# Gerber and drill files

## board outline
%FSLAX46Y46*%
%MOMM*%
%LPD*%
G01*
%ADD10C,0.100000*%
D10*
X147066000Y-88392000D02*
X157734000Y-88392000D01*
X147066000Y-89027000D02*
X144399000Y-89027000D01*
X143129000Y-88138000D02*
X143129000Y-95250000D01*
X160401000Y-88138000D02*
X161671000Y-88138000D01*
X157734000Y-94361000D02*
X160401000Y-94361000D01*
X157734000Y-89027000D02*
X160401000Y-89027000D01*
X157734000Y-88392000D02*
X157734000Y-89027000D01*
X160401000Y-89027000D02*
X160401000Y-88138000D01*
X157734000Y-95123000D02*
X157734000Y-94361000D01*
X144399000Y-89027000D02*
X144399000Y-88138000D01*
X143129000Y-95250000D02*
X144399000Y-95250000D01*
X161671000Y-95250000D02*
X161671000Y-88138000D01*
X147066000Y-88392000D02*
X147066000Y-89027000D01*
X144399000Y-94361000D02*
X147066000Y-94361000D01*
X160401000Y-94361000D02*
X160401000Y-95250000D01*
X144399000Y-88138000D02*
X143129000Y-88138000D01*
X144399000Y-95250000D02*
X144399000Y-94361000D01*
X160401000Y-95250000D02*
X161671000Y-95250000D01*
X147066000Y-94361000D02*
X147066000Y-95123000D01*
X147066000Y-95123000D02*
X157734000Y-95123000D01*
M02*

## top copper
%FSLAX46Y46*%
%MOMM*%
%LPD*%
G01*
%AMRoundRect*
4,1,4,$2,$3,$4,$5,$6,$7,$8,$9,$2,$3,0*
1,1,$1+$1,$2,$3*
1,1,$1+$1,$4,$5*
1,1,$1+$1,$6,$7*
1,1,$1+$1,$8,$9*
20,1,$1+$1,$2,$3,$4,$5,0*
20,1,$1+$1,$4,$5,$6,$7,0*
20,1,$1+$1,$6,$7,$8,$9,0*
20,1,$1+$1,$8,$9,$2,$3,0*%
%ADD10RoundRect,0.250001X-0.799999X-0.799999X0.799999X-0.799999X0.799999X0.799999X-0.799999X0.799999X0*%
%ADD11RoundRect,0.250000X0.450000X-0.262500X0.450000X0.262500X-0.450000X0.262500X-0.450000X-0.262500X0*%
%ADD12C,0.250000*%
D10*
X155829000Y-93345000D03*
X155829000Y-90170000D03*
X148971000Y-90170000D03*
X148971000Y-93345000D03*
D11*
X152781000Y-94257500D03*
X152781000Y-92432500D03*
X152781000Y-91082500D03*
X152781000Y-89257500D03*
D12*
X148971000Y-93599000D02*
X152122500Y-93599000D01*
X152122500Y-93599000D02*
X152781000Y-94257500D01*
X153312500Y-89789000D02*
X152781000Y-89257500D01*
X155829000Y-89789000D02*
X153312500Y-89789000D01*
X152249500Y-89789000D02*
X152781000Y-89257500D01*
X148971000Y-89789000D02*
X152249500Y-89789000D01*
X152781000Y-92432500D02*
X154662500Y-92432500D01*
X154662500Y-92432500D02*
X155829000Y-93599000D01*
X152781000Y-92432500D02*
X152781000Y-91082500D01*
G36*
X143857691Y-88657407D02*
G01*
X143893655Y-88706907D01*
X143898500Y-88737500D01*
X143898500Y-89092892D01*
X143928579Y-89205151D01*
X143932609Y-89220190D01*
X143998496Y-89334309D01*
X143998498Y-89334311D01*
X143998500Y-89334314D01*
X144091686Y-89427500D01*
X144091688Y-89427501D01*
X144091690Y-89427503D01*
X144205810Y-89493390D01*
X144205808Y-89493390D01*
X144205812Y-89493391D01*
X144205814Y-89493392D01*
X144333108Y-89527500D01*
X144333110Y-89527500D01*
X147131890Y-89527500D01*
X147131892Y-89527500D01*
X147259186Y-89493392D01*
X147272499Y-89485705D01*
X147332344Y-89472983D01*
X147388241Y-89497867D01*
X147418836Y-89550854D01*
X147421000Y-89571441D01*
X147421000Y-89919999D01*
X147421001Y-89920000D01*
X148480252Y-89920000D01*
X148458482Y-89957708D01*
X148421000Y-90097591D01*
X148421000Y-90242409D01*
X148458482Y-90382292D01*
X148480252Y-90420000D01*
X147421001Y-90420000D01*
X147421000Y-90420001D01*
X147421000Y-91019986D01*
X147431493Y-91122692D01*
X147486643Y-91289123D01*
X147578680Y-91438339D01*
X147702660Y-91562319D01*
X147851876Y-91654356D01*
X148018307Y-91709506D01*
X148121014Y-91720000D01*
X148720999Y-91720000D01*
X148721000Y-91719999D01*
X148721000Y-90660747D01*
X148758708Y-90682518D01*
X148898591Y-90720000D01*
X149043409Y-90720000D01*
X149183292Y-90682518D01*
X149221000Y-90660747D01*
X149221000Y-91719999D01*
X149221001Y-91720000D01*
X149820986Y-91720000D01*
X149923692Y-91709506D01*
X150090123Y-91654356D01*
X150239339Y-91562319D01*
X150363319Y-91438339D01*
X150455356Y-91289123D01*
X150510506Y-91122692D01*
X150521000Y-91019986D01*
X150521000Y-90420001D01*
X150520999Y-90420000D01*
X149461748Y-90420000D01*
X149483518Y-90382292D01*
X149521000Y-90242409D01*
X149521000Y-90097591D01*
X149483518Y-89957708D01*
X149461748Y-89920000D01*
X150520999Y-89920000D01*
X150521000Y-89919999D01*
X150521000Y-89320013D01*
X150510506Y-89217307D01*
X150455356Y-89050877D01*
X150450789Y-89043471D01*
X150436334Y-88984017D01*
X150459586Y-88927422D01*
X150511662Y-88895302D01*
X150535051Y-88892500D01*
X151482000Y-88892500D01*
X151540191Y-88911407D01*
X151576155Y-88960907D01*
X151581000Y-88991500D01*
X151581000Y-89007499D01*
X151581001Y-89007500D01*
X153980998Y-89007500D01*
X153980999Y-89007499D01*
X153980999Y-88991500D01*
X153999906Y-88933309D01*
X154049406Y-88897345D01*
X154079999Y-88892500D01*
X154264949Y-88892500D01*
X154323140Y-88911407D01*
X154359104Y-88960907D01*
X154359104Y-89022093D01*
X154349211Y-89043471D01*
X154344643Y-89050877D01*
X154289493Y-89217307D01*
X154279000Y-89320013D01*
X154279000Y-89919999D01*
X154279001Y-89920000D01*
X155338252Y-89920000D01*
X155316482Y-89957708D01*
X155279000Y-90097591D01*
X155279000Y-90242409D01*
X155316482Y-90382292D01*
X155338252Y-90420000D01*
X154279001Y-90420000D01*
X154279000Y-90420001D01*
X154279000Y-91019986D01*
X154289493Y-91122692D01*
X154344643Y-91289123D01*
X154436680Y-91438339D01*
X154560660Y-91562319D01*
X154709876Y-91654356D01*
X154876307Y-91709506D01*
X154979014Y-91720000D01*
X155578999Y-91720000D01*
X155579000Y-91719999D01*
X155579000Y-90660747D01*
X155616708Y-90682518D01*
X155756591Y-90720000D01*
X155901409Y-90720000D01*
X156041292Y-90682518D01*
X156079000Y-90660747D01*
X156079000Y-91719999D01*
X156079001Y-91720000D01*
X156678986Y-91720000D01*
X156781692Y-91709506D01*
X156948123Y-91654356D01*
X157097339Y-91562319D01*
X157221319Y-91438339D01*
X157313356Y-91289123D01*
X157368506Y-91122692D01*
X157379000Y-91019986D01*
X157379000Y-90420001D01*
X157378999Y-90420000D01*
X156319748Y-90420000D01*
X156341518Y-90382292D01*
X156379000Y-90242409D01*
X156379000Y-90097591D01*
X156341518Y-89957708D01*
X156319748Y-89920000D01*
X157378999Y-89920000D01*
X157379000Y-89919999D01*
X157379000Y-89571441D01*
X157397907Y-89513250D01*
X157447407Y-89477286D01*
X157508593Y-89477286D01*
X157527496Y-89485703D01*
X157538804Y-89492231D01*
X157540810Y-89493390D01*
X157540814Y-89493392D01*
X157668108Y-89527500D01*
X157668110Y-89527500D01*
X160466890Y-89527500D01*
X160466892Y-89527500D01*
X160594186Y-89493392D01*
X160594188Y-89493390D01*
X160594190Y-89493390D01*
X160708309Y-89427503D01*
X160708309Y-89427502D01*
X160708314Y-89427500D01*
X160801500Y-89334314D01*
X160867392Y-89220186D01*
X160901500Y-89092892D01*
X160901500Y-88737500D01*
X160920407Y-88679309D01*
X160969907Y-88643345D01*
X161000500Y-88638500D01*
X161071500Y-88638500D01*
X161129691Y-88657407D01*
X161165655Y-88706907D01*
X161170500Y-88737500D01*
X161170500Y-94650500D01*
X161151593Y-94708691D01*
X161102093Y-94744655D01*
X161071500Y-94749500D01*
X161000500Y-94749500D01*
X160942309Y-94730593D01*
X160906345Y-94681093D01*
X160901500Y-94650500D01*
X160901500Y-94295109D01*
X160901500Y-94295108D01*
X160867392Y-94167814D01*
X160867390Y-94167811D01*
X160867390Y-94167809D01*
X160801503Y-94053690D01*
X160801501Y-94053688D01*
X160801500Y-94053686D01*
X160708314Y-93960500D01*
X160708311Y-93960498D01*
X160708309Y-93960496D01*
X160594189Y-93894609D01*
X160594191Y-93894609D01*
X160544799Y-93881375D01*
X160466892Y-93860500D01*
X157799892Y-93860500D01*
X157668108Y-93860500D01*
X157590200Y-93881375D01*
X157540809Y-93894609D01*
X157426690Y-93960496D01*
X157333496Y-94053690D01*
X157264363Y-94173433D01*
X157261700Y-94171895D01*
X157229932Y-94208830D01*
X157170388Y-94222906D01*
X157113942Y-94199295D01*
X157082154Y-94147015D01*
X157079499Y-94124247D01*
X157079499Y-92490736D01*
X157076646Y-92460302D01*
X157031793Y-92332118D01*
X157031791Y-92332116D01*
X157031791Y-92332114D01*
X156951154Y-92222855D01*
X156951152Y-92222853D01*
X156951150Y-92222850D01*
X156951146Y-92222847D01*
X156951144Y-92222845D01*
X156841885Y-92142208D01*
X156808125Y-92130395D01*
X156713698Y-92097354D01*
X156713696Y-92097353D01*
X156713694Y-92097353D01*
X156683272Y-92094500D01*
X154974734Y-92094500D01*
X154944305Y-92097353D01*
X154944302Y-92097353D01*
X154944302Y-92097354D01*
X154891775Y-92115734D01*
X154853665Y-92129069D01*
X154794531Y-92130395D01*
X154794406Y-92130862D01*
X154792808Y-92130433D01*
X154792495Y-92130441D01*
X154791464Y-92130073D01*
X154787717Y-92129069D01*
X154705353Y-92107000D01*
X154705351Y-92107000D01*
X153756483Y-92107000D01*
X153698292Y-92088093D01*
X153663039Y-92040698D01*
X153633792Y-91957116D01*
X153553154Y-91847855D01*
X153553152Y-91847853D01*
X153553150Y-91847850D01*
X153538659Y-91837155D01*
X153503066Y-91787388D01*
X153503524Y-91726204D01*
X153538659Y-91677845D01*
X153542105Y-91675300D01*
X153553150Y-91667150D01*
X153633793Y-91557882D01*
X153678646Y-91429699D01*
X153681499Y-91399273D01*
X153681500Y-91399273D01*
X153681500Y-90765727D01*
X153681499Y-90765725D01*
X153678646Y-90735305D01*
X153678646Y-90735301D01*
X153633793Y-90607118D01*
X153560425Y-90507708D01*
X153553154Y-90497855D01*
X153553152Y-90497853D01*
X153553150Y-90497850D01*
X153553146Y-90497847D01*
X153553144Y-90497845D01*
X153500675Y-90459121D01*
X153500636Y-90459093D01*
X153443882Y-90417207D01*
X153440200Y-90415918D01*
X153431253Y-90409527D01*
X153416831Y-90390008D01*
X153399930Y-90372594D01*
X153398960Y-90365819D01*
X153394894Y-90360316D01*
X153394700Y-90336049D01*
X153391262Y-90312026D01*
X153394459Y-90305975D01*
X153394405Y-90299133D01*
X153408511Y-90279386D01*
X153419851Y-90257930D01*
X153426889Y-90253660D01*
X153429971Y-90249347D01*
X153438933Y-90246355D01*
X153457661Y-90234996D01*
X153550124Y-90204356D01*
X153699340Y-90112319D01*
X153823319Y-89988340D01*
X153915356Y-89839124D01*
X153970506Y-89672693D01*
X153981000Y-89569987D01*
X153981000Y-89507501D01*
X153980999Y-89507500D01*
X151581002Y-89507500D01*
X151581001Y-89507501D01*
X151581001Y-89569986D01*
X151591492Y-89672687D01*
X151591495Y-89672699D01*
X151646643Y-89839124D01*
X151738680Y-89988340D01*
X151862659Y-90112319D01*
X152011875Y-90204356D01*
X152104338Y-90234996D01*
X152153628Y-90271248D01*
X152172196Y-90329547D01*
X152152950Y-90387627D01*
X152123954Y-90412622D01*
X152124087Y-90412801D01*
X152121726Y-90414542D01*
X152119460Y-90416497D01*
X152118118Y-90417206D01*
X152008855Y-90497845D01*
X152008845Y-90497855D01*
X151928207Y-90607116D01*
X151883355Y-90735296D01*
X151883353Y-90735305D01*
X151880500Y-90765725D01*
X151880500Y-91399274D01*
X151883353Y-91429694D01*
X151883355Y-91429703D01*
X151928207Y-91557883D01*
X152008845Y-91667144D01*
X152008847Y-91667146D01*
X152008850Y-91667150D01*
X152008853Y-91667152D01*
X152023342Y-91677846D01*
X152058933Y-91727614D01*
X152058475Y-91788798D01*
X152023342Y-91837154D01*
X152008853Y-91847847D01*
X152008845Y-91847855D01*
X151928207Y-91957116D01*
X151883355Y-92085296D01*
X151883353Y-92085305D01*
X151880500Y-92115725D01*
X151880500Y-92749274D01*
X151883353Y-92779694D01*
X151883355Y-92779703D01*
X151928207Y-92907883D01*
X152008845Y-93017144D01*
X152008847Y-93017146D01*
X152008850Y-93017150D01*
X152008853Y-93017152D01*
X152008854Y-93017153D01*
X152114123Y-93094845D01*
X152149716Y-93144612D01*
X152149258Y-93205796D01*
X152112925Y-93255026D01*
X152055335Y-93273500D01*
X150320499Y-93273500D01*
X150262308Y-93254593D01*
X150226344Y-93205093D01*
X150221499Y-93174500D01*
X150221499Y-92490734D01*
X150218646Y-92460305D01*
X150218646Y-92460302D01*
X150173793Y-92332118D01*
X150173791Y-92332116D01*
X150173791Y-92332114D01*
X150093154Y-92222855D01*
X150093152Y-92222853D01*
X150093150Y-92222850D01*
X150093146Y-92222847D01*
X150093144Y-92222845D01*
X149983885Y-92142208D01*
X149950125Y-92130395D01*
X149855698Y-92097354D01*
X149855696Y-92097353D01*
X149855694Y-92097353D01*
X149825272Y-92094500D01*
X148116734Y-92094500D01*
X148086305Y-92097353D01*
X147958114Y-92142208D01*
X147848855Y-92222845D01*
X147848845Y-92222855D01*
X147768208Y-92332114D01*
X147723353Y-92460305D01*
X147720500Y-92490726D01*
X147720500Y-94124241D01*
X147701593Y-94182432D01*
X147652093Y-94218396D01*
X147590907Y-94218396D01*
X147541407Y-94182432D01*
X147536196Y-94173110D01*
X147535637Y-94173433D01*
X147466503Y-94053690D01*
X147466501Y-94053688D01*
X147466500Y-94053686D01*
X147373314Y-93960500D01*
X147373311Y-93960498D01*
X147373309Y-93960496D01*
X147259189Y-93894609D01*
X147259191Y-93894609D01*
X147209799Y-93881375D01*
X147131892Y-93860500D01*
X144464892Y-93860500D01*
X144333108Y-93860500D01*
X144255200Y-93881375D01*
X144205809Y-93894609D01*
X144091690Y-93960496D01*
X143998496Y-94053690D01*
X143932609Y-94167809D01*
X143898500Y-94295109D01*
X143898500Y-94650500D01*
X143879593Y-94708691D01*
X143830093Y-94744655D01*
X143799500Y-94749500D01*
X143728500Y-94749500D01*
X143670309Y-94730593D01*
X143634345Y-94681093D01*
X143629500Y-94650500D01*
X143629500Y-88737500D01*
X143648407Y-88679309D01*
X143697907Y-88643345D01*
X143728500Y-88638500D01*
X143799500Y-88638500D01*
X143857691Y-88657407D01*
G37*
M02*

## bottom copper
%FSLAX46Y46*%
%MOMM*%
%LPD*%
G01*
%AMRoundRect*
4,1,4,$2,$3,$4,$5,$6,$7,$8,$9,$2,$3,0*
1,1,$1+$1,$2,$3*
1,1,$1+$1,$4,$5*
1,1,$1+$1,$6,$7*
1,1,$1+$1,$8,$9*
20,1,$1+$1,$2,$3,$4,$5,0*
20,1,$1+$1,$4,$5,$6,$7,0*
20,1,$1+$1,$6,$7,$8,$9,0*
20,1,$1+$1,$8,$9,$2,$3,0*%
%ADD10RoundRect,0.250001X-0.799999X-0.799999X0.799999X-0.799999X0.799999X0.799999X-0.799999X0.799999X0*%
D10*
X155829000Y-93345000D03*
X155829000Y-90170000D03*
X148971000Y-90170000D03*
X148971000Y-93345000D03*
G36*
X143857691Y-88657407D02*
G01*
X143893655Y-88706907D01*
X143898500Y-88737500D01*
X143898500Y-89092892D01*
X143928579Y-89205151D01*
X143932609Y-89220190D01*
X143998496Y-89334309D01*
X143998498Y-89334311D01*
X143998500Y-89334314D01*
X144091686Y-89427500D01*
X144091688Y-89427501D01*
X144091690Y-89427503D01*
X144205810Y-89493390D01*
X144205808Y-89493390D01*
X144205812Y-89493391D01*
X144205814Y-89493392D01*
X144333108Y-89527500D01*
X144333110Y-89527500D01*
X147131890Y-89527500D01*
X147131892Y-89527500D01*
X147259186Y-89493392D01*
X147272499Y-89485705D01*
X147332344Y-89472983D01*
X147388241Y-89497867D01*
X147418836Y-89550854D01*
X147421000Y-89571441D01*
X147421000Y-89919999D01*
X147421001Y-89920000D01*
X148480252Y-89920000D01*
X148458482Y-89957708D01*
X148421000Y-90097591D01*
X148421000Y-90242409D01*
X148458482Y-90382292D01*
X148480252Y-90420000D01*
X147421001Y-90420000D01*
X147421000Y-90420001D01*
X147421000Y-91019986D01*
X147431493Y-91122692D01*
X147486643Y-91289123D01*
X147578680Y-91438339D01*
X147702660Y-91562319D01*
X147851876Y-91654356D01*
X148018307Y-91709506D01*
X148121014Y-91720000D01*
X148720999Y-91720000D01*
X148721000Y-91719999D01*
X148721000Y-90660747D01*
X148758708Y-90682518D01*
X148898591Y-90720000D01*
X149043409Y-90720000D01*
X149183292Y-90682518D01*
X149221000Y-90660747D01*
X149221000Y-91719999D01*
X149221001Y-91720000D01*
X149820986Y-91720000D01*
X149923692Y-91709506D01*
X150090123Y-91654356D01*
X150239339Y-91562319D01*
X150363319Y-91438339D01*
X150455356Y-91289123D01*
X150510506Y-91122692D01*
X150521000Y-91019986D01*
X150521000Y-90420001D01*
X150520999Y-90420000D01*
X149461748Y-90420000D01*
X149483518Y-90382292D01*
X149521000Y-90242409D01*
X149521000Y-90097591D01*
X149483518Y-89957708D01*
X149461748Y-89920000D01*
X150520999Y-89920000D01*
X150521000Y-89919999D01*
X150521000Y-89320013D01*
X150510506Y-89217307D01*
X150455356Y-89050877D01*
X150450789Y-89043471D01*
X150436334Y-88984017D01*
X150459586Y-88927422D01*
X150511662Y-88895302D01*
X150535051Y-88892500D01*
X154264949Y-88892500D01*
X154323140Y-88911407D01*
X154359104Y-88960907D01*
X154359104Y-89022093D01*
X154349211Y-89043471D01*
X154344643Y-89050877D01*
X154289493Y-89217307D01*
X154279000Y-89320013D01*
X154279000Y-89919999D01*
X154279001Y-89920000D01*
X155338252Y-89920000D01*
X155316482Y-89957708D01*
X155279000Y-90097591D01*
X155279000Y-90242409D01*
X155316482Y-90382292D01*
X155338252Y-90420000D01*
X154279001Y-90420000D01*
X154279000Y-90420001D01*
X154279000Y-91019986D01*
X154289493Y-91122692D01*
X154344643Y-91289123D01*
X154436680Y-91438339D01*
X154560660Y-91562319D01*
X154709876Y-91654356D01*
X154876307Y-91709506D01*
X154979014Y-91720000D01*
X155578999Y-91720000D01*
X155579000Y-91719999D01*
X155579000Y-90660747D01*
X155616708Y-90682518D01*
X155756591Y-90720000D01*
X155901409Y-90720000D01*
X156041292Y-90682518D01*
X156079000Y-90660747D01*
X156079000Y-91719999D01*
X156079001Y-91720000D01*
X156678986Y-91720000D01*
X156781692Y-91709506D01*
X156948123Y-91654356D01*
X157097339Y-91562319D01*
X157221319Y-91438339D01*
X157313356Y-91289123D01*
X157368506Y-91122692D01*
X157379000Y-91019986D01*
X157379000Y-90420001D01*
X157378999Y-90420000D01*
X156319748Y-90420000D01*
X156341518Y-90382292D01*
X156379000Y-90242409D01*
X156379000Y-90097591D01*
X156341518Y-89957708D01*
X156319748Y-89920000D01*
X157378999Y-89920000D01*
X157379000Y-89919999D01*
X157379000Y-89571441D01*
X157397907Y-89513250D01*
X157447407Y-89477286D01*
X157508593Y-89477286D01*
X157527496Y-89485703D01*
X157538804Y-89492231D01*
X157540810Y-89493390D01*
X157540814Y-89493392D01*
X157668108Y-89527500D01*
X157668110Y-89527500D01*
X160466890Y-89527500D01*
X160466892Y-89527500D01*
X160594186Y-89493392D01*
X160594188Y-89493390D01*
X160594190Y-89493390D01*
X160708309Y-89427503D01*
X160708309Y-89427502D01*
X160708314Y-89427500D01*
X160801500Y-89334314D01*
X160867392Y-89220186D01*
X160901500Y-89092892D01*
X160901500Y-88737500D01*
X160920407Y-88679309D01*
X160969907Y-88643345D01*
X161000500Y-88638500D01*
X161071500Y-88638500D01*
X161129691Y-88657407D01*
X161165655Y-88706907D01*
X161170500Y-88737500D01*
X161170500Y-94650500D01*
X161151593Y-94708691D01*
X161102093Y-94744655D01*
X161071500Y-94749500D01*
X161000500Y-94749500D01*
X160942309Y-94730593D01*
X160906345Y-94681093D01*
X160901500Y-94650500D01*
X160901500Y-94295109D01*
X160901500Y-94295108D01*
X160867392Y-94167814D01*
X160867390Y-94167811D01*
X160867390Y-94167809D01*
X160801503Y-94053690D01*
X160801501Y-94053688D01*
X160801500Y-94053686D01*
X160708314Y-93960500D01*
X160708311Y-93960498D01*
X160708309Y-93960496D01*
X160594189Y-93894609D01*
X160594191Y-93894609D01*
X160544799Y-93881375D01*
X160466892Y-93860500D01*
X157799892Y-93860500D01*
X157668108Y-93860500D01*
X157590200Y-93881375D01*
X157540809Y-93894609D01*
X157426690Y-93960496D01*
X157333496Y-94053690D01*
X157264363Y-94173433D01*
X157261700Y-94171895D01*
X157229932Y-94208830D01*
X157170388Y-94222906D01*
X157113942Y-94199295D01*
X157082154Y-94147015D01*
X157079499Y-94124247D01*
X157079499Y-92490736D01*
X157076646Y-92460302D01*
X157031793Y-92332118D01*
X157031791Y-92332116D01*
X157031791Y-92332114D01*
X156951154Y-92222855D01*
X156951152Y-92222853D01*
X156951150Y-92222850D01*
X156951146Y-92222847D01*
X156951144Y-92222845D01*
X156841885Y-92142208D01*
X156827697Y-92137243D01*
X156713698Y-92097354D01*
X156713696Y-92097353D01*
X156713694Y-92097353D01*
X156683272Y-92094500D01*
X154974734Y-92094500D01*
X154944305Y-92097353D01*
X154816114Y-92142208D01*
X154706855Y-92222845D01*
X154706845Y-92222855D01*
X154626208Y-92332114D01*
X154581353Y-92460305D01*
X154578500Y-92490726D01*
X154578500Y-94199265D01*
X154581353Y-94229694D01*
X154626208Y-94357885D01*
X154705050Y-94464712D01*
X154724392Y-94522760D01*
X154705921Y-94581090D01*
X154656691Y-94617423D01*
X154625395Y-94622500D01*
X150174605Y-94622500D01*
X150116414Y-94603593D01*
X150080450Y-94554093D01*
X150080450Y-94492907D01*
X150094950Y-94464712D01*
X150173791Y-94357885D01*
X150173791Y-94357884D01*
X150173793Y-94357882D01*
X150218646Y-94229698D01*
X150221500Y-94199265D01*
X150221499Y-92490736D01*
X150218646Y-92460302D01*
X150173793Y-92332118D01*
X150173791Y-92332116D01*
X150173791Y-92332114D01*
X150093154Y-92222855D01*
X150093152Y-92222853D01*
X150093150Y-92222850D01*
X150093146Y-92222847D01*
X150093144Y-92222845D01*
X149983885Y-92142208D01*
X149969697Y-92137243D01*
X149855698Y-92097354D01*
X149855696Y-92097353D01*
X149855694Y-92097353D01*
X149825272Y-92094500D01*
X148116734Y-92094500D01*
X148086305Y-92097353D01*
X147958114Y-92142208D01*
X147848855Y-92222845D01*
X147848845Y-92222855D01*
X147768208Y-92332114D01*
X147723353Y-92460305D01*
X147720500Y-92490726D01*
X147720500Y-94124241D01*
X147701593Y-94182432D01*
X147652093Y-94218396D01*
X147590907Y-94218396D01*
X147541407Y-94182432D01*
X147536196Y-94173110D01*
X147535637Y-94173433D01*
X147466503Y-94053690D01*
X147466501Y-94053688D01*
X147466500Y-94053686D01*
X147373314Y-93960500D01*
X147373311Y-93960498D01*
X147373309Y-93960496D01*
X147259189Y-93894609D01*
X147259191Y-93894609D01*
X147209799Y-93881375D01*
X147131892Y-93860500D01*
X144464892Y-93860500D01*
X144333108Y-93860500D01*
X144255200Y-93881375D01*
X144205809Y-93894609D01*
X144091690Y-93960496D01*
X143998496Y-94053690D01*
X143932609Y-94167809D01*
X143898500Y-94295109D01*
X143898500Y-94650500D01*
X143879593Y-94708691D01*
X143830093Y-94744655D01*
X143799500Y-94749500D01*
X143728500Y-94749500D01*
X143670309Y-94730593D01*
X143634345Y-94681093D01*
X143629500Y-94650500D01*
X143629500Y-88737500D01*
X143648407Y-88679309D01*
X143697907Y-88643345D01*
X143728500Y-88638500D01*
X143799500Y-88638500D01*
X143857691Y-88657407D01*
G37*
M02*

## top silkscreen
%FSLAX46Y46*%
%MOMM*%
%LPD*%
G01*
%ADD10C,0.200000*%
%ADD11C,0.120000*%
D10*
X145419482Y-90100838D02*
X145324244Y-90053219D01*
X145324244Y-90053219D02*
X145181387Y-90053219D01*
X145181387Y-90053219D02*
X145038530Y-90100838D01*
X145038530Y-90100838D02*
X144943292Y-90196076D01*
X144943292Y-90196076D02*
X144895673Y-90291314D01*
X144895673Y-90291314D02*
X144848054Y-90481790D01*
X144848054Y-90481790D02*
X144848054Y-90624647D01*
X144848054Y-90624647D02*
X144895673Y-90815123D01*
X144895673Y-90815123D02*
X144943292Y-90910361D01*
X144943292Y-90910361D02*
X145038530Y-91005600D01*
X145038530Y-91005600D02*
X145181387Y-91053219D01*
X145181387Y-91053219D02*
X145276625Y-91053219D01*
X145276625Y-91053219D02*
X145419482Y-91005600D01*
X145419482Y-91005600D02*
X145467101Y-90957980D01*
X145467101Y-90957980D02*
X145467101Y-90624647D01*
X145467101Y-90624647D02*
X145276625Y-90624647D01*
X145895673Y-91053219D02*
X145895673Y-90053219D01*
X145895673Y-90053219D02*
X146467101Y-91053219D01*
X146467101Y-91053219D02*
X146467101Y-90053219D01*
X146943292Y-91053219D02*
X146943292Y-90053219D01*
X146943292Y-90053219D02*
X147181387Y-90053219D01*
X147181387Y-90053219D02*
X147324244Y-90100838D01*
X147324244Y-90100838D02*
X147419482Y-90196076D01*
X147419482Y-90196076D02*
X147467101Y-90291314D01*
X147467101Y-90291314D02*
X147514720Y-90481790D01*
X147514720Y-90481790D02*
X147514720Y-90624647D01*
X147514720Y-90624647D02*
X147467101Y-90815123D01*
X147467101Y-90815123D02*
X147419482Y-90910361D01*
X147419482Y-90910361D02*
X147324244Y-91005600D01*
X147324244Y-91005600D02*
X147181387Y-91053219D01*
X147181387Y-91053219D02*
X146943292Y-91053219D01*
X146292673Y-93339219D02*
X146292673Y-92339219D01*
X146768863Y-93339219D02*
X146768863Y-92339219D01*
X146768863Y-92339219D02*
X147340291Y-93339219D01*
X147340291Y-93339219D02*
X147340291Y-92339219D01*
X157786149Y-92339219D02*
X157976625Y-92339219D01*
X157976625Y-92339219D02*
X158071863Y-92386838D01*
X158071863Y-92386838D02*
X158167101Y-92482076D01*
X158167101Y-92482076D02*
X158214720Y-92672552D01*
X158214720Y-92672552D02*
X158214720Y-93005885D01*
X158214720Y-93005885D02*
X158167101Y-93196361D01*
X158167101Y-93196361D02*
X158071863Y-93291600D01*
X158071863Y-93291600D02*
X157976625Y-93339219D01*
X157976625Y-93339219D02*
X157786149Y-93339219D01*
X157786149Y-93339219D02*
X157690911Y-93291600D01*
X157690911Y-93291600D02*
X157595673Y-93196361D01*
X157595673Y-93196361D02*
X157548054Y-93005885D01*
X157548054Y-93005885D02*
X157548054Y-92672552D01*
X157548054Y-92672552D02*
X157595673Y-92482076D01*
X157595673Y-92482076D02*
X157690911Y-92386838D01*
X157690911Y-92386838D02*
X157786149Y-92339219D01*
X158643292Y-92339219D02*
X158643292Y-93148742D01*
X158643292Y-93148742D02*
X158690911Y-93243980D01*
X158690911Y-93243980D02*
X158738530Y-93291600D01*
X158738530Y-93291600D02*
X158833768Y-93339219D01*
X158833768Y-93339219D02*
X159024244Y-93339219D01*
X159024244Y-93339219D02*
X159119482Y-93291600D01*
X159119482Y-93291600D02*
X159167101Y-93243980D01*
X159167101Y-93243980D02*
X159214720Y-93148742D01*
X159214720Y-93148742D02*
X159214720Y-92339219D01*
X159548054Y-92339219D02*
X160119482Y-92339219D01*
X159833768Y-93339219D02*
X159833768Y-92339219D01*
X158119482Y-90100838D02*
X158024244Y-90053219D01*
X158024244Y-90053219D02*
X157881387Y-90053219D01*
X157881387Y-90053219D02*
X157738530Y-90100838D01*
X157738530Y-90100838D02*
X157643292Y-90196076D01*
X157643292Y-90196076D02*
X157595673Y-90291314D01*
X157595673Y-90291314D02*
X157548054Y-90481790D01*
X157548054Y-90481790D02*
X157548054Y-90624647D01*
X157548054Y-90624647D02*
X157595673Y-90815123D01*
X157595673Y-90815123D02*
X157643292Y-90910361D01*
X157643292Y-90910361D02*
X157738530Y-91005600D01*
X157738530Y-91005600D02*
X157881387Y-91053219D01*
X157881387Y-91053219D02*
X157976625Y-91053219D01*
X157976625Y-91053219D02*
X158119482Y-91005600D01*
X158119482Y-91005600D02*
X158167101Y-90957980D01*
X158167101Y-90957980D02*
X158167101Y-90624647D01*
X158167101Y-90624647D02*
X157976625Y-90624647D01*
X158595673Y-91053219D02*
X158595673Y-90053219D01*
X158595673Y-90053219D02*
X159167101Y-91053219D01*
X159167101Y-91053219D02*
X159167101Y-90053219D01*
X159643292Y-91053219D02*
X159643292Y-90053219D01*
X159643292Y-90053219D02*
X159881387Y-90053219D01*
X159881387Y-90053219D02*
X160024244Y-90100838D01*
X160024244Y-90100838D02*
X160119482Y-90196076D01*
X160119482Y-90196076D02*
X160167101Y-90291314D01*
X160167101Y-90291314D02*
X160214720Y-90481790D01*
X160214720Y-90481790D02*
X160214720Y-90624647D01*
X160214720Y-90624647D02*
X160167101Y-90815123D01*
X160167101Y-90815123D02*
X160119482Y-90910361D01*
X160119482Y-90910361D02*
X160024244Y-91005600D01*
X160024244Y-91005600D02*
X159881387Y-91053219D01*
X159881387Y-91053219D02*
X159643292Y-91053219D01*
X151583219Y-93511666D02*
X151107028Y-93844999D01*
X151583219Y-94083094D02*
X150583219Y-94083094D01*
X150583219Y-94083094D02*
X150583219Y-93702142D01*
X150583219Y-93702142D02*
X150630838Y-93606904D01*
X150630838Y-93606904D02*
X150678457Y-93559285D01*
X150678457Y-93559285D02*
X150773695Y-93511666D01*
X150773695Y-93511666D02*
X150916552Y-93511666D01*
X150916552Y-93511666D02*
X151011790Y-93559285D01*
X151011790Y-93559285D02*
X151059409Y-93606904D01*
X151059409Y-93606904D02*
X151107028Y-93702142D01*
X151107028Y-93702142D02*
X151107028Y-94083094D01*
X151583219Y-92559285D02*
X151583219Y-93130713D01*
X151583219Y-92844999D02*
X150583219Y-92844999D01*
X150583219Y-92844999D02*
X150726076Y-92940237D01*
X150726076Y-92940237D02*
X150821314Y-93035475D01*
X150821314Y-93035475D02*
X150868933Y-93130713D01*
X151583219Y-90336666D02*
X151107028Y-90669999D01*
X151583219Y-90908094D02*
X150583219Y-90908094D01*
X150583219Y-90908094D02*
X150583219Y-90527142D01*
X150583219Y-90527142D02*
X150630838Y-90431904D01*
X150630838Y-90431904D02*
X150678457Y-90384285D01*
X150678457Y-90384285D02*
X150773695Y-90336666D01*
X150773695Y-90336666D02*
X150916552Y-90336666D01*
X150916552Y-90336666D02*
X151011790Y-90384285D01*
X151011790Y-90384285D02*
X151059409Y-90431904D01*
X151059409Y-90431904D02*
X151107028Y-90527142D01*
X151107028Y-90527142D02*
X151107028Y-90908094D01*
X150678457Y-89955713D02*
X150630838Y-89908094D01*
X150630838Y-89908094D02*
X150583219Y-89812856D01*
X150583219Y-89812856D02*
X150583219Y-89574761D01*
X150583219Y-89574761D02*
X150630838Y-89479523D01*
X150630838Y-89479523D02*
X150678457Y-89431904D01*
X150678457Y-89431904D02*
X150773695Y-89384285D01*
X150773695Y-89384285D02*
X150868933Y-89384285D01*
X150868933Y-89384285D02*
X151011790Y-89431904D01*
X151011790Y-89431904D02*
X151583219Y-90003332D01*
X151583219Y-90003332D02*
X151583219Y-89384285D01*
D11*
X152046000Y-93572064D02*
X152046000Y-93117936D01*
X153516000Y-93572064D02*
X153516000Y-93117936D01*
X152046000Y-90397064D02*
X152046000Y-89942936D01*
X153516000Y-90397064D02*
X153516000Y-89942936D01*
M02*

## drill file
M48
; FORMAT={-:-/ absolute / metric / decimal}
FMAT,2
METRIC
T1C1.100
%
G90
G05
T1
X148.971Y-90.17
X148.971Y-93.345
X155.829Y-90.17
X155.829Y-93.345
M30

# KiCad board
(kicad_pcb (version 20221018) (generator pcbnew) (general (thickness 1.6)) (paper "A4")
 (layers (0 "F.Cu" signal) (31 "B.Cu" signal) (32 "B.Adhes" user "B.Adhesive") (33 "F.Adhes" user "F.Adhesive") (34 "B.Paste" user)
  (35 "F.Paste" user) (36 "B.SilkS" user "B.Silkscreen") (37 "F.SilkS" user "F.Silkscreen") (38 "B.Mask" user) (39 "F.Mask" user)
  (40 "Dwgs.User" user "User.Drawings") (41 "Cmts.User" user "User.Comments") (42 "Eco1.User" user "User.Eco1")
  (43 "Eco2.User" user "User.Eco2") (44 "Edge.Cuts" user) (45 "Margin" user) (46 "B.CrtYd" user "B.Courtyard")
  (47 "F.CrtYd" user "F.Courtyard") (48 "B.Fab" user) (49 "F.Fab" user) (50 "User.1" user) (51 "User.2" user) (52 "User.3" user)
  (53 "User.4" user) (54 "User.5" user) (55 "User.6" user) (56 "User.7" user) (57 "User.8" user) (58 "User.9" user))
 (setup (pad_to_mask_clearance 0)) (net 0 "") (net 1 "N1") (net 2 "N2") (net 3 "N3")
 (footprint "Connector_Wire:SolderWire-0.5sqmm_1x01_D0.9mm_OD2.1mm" (layer "F.Cu") (at 155.829 93.345)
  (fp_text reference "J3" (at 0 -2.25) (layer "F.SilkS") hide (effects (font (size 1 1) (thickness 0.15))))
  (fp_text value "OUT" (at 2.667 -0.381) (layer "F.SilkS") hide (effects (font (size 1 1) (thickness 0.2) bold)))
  (pad "1" thru_hole roundrect (at 0 0) (size 2.1 2.1) (drill 1.1) (layers "*.Cu" "*.Mask") (roundrect_rratio 0.1190480952) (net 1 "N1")))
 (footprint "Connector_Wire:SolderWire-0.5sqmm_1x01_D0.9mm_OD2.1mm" (layer "F.Cu") (at 155.829 90.17)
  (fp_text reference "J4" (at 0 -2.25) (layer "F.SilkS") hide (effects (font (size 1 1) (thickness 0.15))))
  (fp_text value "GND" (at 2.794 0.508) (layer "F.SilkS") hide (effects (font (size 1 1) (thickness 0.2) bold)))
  (pad "1" thru_hole roundrect (at 0 0) (size 2.1 2.1) (drill 1.1) (layers "*.Cu" "*.Mask") (roundrect_rratio 0.1190480952) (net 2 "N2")))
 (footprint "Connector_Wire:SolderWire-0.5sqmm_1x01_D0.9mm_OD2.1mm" (layer "F.Cu") (at 148.971 90.17)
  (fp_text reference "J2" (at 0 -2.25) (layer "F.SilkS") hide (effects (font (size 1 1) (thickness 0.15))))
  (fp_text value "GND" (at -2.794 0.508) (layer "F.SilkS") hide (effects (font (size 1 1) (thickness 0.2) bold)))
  (pad "1" thru_hole roundrect (at 0 0) (size 2.1 2.1) (drill 1.1) (layers "*.Cu" "*.Mask") (roundrect_rratio 0.1190480952) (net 2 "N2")))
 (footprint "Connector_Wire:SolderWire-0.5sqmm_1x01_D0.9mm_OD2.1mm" (layer "F.Cu") (at 148.971 93.345)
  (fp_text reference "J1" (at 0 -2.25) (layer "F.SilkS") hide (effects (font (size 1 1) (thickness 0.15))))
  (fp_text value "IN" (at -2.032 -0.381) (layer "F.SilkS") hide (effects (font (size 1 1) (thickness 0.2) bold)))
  (pad "1" thru_hole roundrect (at 0 0) (size 2.1 2.1) (drill 1.1) (layers "*.Cu" "*.Mask") (roundrect_rratio 0.1190480952) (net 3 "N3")))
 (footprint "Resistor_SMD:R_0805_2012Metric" (layer "F.Cu") (at 152.781 93.345 90)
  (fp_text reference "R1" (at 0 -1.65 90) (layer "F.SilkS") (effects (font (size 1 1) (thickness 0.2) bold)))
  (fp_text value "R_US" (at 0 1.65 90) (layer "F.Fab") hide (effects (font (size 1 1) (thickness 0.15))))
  (fp_line (start -0.227064 -0.735) (end 0.227064 -0.735) (stroke (width 0.12) (type solid)) (layer "F.SilkS"))
  (fp_line (start -0.227064 0.735) (end 0.227064 0.735) (stroke (width 0.12) (type solid)) (layer "F.SilkS"))
  (pad "1" smd roundrect (at -0.9125 0 90) (size 1.025 1.4) (layers "F.Cu" "F.Paste" "F.Mask") (roundrect_rratio 0.243902439) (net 3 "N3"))
  (pad "2" smd roundrect (at 0.9125 0 90) (size 1.025 1.4) (layers "F.Cu" "F.Paste" "F.Mask") (roundrect_rratio 0.243902439) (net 1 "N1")))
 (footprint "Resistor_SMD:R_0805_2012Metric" (layer "F.Cu") (at 152.781 90.17 90)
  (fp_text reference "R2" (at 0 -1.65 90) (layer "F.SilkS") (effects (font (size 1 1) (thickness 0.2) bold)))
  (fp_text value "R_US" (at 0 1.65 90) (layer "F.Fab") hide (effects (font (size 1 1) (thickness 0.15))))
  (fp_line (start -0.227064 -0.735) (end 0.227064 -0.735) (stroke (width 0.12) (type solid)) (layer "F.SilkS"))
  (fp_line (start -0.227064 0.735) (end 0.227064 0.735) (stroke (width 0.12) (type solid)) (layer "F.SilkS"))
  (pad "1" smd roundrect (at -0.9125 0 90) (size 1.025 1.4) (layers "F.Cu" "F.Paste" "F.Mask") (roundrect_rratio 0.243902439) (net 1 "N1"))
  (pad "2" smd roundrect (at 0.9125 0 90) (size 1.025 1.4) (layers "F.Cu" "F.Paste" "F.Mask") (roundrect_rratio 0.243902439) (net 2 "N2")))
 (gr_line (start 147.066 88.392) (end 157.734 88.392) (stroke (width 0.1) (type default)) (layer "Edge.Cuts"))
 (gr_line (start 147.066 89.027) (end 144.399 89.027) (stroke (width 0.1) (type default)) (layer "Edge.Cuts"))
 (gr_line (start 143.129 88.138) (end 143.129 95.25) (stroke (width 0.1) (type default)) (layer "Edge.Cuts"))
 (gr_line (start 160.401 88.138) (end 161.671 88.138) (stroke (width 0.1) (type default)) (layer "Edge.Cuts"))
 (gr_line (start 157.734 94.361) (end 160.401 94.361) (stroke (width 0.1) (type default)) (layer "Edge.Cuts"))
 (gr_line (start 157.734 89.027) (end 160.401 89.027) (stroke (width 0.1) (type default)) (layer "Edge.Cuts"))
 (gr_line (start 157.734 88.392) (end 157.734 89.027) (stroke (width 0.1) (type default)) (layer "Edge.Cuts"))
 (gr_line (start 160.401 89.027) (end 160.401 88.138) (stroke (width 0.1) (type default)) (layer "Edge.Cuts"))
 (gr_line (start 157.734 95.123) (end 157.734 94.361) (stroke (width 0.1) (type default)) (layer "Edge.Cuts"))
 (gr_line (start 144.399 89.027) (end 144.399 88.138) (stroke (width 0.1) (type default)) (layer "Edge.Cuts"))
 (gr_line (start 143.129 95.25) (end 144.399 95.25) (stroke (width 0.1) (type default)) (layer "Edge.Cuts"))
 (gr_line (start 161.671 95.25) (end 161.671 88.138) (stroke (width 0.1) (type default)) (layer "Edge.Cuts"))
 (gr_line (start 147.066 88.392) (end 147.066 89.027) (stroke (width 0.1) (type default)) (layer "Edge.Cuts"))
 (gr_line (start 144.399 94.361) (end 147.066 94.361) (stroke (width 0.1) (type default)) (layer "Edge.Cuts"))
 (gr_line (start 160.401 94.361) (end 160.401 95.25) (stroke (width 0.1) (type default)) (layer "Edge.Cuts"))
 (gr_line (start 144.399 88.138) (end 143.129 88.138) (stroke (width 0.1) (type default)) (layer "Edge.Cuts"))
 (gr_line (start 144.399 95.25) (end 144.399 94.361) (stroke (width 0.1) (type default)) (layer "Edge.Cuts"))
 (gr_line (start 160.401 95.25) (end 161.671 95.25) (stroke (width 0.1) (type default)) (layer "Edge.Cuts"))
 (gr_line (start 147.066 94.361) (end 147.066 95.123) (stroke (width 0.1) (type default)) (layer "Edge.Cuts"))
 (gr_line (start 147.066 95.123) (end 157.734 95.123) (stroke (width 0.1) (type default)) (layer "Edge.Cuts"))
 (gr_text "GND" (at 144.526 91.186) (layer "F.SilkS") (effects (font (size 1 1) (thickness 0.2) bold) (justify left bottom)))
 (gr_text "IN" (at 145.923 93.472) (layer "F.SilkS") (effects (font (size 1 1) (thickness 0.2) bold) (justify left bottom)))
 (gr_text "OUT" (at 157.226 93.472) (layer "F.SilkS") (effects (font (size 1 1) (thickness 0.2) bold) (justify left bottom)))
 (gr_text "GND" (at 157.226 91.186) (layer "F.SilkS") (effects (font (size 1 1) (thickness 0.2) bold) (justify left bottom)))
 (segment (start 148.971 93.599) (end 152.1225 93.599) (width 0.25) (layer "F.Cu") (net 3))
 (segment (start 152.1225 93.599) (end 152.781 94.2575) (width 0.25) (layer "F.Cu") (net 3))
 (segment (start 153.3125 89.789) (end 152.781 89.2575) (width 0.25) (layer "F.Cu") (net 2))
 (segment (start 155.829 89.789) (end 153.3125 89.789) (width 0.25) (layer "F.Cu") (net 2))
 (segment (start 152.2495 89.789) (end 152.781 89.2575) (width 0.25) (layer "F.Cu") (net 2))
 (segment (start 148.971 89.789) (end 152.2495 89.789) (width 0.25) (layer "F.Cu") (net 2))
 (segment (start 152.781 92.4325) (end 154.6625 92.4325) (width 0.25) (layer "F.Cu") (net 1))
 (segment (start 154.6625 92.4325) (end 155.829 93.599) (width 0.25) (layer "F.Cu") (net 1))
 (segment (start 152.781 92.4325) (end 152.781 91.0825) (width 0.25) (layer "F.Cu") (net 1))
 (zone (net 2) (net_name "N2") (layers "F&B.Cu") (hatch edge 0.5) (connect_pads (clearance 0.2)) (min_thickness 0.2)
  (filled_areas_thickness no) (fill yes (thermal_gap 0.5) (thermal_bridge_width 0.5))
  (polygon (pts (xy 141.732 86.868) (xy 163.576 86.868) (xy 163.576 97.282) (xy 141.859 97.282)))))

